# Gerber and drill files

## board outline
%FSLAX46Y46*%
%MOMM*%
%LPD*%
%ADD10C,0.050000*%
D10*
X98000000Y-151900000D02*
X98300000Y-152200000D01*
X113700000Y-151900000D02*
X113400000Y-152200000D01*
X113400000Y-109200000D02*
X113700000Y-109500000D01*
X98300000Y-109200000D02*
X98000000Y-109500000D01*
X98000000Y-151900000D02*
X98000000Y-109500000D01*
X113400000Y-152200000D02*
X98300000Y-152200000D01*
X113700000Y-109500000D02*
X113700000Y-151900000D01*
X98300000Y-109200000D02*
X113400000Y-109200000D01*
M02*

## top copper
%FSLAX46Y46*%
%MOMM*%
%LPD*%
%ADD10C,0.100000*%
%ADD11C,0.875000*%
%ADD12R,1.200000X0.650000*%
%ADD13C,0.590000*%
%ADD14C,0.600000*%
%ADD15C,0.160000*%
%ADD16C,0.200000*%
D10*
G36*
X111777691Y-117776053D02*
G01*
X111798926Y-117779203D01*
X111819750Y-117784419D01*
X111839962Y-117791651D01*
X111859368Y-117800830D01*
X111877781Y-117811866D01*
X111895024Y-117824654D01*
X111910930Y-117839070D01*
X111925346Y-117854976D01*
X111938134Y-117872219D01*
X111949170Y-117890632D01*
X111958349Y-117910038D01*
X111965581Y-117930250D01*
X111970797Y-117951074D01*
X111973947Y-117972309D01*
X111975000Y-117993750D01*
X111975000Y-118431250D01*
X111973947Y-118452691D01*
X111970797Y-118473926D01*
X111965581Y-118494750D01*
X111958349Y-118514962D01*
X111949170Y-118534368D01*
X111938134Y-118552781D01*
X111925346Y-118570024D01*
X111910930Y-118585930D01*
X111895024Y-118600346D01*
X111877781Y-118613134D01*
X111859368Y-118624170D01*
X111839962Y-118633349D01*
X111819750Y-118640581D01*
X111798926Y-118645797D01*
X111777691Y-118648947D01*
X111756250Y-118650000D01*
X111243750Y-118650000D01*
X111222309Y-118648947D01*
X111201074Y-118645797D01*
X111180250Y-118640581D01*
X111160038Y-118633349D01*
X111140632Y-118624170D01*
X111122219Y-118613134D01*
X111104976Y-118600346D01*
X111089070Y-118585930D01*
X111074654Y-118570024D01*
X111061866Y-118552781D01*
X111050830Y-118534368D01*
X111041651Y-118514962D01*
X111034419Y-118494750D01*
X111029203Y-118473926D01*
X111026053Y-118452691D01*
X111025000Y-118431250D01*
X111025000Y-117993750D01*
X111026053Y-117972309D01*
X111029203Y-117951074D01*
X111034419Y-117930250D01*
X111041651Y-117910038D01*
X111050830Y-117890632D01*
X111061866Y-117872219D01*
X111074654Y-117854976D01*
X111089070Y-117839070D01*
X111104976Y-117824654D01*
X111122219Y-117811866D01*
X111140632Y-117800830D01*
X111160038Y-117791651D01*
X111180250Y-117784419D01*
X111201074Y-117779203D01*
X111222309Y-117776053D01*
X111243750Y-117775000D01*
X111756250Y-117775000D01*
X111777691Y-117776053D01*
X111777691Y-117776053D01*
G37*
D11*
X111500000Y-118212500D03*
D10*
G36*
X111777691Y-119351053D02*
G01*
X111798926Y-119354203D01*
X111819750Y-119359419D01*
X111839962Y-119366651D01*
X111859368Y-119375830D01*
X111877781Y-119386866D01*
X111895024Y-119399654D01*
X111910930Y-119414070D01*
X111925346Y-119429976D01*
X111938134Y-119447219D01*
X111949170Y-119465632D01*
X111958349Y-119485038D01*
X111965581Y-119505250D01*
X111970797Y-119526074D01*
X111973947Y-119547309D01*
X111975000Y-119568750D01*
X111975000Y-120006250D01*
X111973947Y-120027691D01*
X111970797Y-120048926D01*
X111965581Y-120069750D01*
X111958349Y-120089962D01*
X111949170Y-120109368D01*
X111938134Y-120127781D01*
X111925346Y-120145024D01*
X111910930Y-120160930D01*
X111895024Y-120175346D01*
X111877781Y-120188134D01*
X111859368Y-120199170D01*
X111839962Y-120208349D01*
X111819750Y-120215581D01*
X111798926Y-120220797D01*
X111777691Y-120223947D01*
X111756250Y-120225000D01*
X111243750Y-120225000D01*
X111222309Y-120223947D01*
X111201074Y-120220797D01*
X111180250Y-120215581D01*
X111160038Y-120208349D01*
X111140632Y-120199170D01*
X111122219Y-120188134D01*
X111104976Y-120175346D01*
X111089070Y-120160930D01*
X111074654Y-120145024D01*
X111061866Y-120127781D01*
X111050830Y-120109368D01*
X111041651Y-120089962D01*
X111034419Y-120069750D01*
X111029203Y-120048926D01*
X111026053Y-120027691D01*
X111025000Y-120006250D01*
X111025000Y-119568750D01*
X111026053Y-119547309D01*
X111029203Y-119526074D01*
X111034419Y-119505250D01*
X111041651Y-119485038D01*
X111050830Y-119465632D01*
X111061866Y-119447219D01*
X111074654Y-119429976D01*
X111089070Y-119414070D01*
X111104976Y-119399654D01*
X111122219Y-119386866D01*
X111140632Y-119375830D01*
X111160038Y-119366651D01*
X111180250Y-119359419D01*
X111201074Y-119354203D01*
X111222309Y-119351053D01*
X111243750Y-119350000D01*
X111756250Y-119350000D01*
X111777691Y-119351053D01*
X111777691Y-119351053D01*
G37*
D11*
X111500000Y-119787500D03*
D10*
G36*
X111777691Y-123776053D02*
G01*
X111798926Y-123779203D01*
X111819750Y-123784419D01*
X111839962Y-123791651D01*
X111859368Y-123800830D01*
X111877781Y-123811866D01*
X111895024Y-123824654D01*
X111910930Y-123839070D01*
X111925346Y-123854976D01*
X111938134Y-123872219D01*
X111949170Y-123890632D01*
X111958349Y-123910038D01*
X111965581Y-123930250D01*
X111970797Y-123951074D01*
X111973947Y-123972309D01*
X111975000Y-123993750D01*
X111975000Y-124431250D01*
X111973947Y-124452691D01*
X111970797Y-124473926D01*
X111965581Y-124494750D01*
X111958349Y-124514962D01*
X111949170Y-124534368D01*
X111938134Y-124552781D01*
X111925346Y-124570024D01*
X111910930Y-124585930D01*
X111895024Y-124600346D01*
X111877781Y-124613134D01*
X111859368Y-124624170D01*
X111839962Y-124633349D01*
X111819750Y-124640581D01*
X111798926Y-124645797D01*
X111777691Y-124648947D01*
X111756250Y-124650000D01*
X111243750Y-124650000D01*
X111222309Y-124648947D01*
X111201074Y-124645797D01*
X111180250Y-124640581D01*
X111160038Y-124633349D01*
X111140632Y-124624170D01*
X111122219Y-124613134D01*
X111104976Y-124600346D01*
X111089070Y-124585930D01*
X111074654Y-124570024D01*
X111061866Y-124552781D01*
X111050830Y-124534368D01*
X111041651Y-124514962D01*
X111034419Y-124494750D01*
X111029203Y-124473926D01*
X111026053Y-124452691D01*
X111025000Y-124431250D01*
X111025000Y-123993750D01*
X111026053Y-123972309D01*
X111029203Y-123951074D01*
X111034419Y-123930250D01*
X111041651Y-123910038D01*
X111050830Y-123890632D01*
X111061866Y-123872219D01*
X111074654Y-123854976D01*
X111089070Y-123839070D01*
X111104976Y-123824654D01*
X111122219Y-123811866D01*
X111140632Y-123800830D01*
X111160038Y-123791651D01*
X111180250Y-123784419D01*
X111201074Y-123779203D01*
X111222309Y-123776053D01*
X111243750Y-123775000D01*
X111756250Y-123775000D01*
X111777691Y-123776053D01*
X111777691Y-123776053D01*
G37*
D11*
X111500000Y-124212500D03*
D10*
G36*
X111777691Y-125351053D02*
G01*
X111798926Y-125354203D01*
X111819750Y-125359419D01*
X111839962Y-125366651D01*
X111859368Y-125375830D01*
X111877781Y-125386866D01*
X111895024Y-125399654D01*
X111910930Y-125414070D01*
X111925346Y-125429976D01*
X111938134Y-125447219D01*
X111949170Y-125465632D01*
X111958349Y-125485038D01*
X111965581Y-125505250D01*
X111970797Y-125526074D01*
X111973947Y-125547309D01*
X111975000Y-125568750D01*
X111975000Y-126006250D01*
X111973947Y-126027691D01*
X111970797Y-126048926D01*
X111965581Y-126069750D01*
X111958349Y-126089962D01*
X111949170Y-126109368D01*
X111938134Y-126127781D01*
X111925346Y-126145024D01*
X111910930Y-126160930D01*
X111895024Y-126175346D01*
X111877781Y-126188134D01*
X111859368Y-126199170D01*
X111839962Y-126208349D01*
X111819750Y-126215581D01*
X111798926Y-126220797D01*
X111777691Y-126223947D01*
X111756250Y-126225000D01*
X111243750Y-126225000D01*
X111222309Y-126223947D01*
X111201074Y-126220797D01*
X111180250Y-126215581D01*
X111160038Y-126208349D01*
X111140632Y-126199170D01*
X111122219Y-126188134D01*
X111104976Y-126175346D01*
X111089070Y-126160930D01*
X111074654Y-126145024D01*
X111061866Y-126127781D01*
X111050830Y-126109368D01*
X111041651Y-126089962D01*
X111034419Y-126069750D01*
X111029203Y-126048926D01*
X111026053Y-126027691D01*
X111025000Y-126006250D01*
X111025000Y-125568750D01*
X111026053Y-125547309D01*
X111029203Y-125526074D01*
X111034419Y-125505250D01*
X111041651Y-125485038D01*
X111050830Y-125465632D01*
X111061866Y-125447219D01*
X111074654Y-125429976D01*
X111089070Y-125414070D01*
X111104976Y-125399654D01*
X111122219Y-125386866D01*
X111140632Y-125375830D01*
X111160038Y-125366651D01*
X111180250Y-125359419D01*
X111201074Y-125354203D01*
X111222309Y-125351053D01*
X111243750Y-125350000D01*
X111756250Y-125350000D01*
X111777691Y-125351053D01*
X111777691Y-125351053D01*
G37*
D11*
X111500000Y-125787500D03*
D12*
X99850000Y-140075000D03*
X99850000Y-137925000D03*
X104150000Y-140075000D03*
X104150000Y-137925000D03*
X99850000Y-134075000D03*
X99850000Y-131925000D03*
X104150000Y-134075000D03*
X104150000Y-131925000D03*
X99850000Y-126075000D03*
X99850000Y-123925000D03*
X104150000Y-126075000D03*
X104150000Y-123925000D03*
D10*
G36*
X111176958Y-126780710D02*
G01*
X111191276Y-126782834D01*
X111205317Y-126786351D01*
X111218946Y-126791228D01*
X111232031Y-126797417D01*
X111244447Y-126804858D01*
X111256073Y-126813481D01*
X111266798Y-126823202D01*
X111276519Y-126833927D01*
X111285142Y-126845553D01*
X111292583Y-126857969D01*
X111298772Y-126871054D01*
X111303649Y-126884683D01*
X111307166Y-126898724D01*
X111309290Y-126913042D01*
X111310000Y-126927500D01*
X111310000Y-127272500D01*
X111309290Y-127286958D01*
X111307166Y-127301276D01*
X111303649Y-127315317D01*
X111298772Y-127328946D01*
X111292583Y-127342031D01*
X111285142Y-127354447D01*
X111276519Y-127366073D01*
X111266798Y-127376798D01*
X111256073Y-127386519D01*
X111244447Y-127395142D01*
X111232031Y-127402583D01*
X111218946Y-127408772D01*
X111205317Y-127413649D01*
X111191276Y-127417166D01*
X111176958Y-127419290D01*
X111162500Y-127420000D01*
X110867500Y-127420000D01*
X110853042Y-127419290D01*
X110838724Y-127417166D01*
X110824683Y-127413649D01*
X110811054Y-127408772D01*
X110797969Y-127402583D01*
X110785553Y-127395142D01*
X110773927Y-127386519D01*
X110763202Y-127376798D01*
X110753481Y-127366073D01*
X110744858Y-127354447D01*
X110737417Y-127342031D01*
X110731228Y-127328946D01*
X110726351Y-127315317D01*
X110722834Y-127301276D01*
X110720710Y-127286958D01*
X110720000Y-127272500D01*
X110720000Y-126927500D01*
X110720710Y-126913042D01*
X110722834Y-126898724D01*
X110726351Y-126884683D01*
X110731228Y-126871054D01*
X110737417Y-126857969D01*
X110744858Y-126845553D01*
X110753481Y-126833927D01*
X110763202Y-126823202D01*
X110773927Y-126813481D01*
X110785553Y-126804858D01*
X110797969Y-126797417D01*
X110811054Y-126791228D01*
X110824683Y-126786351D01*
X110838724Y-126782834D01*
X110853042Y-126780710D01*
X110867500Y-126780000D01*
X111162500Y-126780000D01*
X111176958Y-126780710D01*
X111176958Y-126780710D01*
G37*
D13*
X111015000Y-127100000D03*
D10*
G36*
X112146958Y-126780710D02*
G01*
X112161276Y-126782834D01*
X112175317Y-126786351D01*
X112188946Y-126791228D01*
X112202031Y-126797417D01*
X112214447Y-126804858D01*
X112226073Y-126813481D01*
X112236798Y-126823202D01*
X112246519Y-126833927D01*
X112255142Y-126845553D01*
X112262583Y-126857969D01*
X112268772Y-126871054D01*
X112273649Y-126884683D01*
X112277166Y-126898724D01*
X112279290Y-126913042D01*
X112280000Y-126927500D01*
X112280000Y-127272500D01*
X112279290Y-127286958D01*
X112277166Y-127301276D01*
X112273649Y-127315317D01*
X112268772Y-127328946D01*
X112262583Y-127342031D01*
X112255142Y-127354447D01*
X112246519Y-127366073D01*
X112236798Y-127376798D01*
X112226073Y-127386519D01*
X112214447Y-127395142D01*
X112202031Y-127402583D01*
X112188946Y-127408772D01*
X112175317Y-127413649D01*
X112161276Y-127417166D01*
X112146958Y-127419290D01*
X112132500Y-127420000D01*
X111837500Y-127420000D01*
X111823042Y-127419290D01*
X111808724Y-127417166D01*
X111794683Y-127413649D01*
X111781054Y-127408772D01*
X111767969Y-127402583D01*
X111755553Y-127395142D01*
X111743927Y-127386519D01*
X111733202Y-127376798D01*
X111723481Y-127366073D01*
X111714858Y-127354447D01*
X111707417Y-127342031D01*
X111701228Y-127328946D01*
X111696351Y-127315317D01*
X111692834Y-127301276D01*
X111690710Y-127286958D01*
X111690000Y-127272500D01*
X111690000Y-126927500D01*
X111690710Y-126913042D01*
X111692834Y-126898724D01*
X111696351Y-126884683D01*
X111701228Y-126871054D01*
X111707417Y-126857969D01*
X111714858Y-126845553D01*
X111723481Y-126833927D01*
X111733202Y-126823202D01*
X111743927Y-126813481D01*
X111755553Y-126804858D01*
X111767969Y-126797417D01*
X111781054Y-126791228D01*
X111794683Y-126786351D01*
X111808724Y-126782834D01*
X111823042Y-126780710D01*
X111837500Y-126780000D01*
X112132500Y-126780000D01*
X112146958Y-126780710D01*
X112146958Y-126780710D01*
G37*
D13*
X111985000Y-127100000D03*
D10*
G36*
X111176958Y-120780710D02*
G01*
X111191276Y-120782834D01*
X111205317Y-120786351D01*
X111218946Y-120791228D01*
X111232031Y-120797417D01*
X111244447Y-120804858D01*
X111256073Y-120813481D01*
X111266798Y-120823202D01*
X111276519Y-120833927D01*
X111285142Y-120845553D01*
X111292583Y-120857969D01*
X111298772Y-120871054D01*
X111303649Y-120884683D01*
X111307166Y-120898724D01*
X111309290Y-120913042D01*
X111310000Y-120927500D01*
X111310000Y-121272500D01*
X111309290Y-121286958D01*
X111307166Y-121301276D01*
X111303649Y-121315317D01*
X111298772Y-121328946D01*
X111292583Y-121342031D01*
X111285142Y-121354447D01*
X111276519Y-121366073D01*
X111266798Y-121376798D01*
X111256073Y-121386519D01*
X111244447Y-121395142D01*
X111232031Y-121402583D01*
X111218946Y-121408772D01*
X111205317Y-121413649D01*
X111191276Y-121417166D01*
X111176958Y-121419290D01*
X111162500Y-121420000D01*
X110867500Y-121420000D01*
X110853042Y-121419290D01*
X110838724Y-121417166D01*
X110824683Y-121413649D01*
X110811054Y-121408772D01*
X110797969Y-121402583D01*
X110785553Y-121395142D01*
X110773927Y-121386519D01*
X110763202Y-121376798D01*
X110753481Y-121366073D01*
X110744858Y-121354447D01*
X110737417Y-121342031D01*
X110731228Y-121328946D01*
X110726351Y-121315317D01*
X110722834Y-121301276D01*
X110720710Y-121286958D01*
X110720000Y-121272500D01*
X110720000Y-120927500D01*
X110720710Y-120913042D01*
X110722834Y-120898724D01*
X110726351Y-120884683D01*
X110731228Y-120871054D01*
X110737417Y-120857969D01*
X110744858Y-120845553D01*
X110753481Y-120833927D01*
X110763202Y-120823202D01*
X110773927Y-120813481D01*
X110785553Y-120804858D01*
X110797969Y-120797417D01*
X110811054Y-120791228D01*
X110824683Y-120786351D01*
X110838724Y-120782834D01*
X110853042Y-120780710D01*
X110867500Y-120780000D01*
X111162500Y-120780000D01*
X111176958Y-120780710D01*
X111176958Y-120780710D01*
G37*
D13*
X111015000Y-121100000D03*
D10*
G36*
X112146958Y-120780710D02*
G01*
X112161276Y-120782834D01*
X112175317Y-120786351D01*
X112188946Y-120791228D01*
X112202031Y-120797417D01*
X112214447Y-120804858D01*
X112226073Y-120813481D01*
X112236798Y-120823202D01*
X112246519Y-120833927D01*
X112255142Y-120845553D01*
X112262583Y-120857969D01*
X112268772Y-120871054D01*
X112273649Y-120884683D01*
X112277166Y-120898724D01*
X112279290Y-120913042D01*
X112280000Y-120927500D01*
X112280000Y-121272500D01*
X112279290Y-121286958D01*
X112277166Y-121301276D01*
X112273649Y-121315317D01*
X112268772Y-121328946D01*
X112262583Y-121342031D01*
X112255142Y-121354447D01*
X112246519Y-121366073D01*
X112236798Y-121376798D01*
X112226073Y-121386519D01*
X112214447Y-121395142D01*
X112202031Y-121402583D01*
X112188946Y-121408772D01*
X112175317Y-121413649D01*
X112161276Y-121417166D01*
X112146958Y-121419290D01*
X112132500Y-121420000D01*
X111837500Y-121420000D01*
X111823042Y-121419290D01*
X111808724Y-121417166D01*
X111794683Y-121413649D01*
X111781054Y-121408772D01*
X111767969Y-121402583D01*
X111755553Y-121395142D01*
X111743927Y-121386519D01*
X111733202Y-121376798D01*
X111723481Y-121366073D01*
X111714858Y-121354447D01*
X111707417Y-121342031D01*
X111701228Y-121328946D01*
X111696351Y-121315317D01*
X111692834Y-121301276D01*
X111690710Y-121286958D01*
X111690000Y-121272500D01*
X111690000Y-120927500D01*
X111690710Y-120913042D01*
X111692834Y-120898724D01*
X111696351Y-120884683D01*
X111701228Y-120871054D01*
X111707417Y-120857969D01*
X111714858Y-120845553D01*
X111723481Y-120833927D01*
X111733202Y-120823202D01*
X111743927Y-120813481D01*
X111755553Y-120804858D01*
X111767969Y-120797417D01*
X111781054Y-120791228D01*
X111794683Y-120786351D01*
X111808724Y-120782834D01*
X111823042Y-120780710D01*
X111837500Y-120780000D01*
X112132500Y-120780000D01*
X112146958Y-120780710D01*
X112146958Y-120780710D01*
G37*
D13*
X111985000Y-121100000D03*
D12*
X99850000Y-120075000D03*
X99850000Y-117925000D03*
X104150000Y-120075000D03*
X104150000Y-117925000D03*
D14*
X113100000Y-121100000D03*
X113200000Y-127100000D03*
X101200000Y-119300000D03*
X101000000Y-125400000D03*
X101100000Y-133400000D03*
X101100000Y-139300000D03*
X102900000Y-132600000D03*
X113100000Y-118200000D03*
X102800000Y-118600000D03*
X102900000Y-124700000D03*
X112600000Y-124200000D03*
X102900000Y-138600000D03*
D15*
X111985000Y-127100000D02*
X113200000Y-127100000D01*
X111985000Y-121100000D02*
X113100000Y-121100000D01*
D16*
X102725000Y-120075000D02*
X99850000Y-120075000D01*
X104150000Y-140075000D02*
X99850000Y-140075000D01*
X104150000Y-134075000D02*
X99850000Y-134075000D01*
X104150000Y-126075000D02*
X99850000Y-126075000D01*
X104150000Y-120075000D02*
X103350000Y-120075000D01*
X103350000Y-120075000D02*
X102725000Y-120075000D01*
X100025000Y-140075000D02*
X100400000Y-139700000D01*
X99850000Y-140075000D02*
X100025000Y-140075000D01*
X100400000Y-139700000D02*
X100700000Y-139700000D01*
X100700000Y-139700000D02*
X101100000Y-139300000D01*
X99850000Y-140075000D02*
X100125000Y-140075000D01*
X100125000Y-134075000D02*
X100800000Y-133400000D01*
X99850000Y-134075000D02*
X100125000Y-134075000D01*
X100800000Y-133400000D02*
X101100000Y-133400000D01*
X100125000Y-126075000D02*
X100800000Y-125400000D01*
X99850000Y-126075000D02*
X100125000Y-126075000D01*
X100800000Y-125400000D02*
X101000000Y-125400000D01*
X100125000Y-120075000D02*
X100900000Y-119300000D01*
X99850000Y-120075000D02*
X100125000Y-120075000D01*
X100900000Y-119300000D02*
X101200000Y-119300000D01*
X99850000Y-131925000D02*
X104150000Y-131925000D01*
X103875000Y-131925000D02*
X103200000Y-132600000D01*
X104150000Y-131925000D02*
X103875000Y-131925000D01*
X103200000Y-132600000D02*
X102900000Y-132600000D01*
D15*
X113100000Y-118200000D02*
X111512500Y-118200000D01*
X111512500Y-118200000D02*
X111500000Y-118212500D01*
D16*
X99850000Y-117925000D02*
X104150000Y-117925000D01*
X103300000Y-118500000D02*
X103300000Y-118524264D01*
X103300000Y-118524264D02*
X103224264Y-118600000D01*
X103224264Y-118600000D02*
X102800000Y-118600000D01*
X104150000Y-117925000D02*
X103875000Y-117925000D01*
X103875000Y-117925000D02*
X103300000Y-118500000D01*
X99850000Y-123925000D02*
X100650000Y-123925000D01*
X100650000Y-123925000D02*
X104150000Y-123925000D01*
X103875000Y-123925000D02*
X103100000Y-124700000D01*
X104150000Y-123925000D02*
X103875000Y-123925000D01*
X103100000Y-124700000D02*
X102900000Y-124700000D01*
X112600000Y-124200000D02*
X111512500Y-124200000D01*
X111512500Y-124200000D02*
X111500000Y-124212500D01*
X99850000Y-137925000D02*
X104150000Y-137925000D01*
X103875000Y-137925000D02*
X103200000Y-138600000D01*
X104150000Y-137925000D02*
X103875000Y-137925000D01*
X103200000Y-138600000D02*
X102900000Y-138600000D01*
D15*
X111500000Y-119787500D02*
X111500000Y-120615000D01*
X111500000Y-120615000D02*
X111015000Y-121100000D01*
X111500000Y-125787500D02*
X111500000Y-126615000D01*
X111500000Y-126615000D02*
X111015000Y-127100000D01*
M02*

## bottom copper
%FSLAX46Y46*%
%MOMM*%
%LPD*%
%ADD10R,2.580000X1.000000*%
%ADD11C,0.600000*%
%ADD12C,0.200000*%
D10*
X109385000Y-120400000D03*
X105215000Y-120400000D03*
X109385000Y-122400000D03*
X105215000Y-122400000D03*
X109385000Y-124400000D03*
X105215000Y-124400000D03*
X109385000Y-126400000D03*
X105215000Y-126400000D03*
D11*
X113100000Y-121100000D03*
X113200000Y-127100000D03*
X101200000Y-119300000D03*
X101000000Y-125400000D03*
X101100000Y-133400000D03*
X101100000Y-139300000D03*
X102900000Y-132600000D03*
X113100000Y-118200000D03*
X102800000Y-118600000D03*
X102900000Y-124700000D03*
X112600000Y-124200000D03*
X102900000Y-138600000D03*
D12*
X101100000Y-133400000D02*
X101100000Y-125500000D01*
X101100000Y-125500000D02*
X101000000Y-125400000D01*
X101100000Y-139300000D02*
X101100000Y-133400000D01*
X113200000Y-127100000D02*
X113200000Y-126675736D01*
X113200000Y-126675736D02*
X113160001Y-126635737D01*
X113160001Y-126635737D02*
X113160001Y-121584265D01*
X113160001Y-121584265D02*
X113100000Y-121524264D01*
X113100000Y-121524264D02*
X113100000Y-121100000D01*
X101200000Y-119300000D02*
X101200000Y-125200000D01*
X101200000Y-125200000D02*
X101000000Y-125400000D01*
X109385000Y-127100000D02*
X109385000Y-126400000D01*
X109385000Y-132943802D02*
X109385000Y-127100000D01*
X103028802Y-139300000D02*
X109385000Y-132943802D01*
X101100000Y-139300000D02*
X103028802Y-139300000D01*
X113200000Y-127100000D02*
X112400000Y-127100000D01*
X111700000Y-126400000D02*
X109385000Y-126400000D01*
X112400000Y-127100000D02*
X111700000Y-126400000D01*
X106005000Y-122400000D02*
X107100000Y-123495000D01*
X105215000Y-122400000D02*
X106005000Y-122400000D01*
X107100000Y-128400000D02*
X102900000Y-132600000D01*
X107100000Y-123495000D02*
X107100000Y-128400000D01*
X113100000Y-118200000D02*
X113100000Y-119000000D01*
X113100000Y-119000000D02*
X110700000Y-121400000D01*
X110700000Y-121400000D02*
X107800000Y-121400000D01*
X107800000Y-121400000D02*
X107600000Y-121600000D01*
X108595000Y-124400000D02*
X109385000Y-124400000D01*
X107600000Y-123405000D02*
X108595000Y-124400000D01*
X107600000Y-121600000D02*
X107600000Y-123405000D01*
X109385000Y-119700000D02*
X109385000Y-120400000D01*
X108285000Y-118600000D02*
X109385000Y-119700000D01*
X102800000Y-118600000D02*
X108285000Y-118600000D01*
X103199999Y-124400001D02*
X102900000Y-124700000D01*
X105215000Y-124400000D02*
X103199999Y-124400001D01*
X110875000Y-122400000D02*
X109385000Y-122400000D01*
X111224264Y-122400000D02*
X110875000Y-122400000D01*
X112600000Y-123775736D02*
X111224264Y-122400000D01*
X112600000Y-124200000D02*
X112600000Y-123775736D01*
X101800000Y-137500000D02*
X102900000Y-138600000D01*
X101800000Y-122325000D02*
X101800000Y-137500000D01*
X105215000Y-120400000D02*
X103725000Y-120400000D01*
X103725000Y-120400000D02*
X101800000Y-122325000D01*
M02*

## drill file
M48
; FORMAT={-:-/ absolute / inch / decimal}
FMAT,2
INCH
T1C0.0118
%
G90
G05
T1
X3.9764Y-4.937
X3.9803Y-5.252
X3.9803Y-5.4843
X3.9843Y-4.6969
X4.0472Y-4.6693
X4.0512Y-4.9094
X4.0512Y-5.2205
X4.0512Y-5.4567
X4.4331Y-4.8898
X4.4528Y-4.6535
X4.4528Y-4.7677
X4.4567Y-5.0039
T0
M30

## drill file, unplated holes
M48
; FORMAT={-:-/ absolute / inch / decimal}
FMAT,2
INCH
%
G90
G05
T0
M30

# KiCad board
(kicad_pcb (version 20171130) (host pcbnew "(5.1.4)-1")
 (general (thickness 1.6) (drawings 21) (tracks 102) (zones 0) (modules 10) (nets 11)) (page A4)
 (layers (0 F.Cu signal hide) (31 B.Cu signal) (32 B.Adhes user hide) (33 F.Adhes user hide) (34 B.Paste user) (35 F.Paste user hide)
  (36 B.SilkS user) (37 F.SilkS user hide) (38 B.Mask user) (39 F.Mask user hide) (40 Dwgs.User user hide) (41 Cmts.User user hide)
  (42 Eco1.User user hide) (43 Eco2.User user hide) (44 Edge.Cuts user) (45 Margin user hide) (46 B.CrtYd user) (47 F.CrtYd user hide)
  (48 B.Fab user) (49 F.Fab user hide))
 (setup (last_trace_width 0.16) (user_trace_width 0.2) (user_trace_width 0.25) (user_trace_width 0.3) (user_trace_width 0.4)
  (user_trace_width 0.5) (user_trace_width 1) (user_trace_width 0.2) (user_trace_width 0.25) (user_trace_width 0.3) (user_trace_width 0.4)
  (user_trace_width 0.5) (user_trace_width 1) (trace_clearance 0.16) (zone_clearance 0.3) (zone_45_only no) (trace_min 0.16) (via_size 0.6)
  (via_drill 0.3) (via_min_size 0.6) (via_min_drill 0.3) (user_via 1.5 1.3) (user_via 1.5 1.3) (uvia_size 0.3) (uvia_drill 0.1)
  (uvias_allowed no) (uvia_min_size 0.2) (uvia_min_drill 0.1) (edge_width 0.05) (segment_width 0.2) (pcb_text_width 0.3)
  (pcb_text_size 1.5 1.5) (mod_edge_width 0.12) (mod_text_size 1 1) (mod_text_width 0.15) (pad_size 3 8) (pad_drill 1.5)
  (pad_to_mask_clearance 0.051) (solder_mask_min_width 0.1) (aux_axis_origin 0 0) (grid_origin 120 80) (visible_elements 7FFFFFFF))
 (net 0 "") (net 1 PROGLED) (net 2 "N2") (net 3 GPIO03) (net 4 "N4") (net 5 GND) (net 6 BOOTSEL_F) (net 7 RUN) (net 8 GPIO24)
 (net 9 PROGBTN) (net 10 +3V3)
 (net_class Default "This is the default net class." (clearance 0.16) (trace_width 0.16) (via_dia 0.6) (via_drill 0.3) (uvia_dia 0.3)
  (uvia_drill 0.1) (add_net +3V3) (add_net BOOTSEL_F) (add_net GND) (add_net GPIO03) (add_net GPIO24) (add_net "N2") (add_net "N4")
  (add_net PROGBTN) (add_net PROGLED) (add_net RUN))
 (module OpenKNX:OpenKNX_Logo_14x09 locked (layer F.Cu) (at 105.8 146.4)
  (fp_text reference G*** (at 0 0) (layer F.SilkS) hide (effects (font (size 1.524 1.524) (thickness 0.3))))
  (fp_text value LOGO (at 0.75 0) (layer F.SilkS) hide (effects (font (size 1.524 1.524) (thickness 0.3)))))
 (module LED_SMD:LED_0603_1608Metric (layer F.Cu) (at 111.5 119 90)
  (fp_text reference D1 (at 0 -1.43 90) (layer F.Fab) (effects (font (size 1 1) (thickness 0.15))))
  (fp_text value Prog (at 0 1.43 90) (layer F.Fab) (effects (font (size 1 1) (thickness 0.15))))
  (pad 2 smd roundrect (at 0.7875 0 90) (size 0.875 0.95) (layers F.Cu F.Paste F.Mask) (roundrect_rratio 0.25) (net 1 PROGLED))
  (pad 1 smd roundrect (at -0.7875 0 90) (size 0.875 0.95) (layers F.Cu F.Paste F.Mask) (roundrect_rratio 0.25) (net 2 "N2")))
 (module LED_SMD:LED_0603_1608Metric (layer F.Cu) (at 111.5 125 90)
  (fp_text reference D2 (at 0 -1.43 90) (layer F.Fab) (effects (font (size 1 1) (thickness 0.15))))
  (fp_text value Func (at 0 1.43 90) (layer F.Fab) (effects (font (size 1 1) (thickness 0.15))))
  (pad 2 smd roundrect (at 0.7875 0 90) (size 0.875 0.95) (layers F.Cu F.Paste F.Mask) (roundrect_rratio 0.25) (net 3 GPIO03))
  (pad 1 smd roundrect (at -0.7875 0 90) (size 0.875 0.95) (layers F.Cu F.Paste F.Mask) (roundrect_rratio 0.25) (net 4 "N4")))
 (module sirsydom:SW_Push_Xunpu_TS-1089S (layer F.Cu) (at 102 139)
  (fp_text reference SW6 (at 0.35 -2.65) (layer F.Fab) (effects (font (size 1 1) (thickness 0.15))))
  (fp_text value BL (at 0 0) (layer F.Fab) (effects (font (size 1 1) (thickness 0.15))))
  (pad 2 smd rect (at -2.15 1.075) (size 1.2 0.65) (layers F.Cu F.Paste F.Mask) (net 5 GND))
  (pad 1 smd rect (at -2.15 -1.075) (size 1.2 0.65) (layers F.Cu F.Paste F.Mask) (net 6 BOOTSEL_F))
  (pad 2 smd rect (at 2.15 1.075) (size 1.2 0.65) (layers F.Cu F.Paste F.Mask) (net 5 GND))
  (pad 1 smd rect (at 2.15 -1.075) (size 1.2 0.65) (layers F.Cu F.Paste F.Mask) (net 6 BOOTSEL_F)))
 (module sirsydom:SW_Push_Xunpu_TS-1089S (layer F.Cu) (at 102 133)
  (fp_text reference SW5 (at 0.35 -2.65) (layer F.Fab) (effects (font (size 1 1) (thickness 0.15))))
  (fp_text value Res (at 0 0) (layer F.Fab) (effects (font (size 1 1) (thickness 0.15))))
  (pad 2 smd rect (at -2.15 1.075) (size 1.2 0.65) (layers F.Cu F.Paste F.Mask) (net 5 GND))
  (pad 1 smd rect (at -2.15 -1.075) (size 1.2 0.65) (layers F.Cu F.Paste F.Mask) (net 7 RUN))
  (pad 2 smd rect (at 2.15 1.075) (size 1.2 0.65) (layers F.Cu F.Paste F.Mask) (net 5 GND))
  (pad 1 smd rect (at 2.15 -1.075) (size 1.2 0.65) (layers F.Cu F.Paste F.Mask) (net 7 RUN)))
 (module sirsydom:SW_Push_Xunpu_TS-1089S (layer F.Cu) (at 102 125)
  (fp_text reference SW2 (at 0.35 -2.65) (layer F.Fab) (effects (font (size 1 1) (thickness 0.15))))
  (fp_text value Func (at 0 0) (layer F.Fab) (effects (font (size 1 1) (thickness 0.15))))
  (pad 2 smd rect (at -2.15 1.075) (size 1.2 0.65) (layers F.Cu F.Paste F.Mask) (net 5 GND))
  (pad 1 smd rect (at -2.15 -1.075) (size 1.2 0.65) (layers F.Cu F.Paste F.Mask) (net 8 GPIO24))
  (pad 2 smd rect (at 2.15 1.075) (size 1.2 0.65) (layers F.Cu F.Paste F.Mask) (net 5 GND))
  (pad 1 smd rect (at 2.15 -1.075) (size 1.2 0.65) (layers F.Cu F.Paste F.Mask) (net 8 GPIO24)))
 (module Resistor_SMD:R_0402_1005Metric (layer F.Cu) (at 111.5 127.1 180)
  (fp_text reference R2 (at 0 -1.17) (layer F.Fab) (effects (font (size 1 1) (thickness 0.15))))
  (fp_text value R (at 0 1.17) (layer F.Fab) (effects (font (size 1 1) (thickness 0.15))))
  (pad 2 smd roundrect (at 0.485 0 180) (size 0.59 0.64) (layers F.Cu F.Paste F.Mask) (roundrect_rratio 0.25) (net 4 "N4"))
  (pad 1 smd roundrect (at -0.485 0 180) (size 0.59 0.64) (layers F.Cu F.Paste F.Mask) (roundrect_rratio 0.25) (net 5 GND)))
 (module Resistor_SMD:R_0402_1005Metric (layer F.Cu) (at 111.5 121.1 180)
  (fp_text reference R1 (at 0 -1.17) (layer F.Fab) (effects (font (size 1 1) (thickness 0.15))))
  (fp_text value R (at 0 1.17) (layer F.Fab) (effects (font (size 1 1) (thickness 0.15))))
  (pad 2 smd roundrect (at 0.485 0 180) (size 0.59 0.64) (layers F.Cu F.Paste F.Mask) (roundrect_rratio 0.25) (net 2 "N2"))
  (pad 1 smd roundrect (at -0.485 0 180) (size 0.59 0.64) (layers F.Cu F.Paste F.Mask) (roundrect_rratio 0.25) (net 5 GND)))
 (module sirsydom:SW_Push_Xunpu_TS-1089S (layer F.Cu) (at 102 119)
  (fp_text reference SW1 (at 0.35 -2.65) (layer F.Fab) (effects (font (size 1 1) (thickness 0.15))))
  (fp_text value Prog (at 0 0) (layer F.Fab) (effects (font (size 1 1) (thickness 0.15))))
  (pad 2 smd rect (at -2.15 1.075) (size 1.2 0.65) (layers F.Cu F.Paste F.Mask) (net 5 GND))
  (pad 1 smd rect (at -2.15 -1.075) (size 1.2 0.65) (layers F.Cu F.Paste F.Mask) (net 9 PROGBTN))
  (pad 2 smd rect (at 2.15 1.075) (size 1.2 0.65) (layers F.Cu F.Paste F.Mask) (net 5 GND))
  (pad 1 smd rect (at 2.15 -1.075) (size 1.2 0.65) (layers F.Cu F.Paste F.Mask) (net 9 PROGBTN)))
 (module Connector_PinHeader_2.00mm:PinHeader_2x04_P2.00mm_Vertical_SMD (layer B.Cu) (at 107.3 123.4)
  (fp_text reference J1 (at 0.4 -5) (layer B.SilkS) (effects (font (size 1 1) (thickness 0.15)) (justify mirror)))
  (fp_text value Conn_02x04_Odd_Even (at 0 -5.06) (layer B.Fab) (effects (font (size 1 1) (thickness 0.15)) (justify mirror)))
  (pad 8 smd rect (at 2.085 -3) (size 2.58 1) (layers B.Cu B.Paste B.Mask) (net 9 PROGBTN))
  (pad 7 smd rect (at -2.085 -3) (size 2.58 1) (layers B.Cu B.Paste B.Mask) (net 6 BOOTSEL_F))
  (pad 6 smd rect (at 2.085 -1) (size 2.58 1) (layers B.Cu B.Paste B.Mask) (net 3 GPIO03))
  (pad 5 smd rect (at -2.085 -1) (size 2.58 1) (layers B.Cu B.Paste B.Mask) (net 7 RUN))
  (pad 4 smd rect (at 2.085 1) (size 2.58 1) (layers B.Cu B.Paste B.Mask) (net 1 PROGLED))
  (pad 3 smd rect (at -2.085 1) (size 2.58 1) (layers B.Cu B.Paste B.Mask) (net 8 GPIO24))
  (pad 2 smd rect (at 2.085 3) (size 2.58 1) (layers B.Cu B.Paste B.Mask) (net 5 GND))
  (pad 1 smd rect (at -2.085 3) (size 2.58 1) (layers B.Cu B.Paste B.Mask) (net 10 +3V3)))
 (gr_line (start 98 151.9) (end 98.3 152.2) (layer Edge.Cuts) (width 0.05))
 (gr_line (start 113.7 151.9) (end 113.4 152.2) (layer Edge.Cuts) (width 0.05))
 (gr_line (start 113.4 109.2) (end 113.7 109.5) (layer Edge.Cuts) (width 0.05))
 (gr_line (start 98.3 109.2) (end 98 109.5) (layer Edge.Cuts) (width 0.05))
 (gr_line (start 98 151.9) (end 98 109.5) (layer Edge.Cuts) (width 0.05))
 (gr_line (start 113.4 152.2) (end 98.3 152.2) (layer Edge.Cuts) (width 0.05))
 (gr_line (start 113.7 109.5) (end 113.7 151.9) (layer Edge.Cuts) (width 0.05))
 (gr_line (start 98.3 109.2) (end 113.4 109.2) (layer Edge.Cuts) (width 0.05))
 (segment (start 101.1 133.4) (end 101.1 125.5) (width 0.2) (layer B.Cu) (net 5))
 (segment (start 101.1 125.5) (end 101 125.4) (width 0.2) (layer B.Cu) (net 5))
 (segment (start 101.1 139.3) (end 101.1 133.4) (width 0.2) (layer B.Cu) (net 5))
 (segment (start 113.2 127.1) (end 113.2 126.675736) (width 0.2) (layer B.Cu) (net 5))
 (segment (start 113.2 126.675736) (end 113.160001 126.635737) (width 0.2) (layer B.Cu) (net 5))
 (segment (start 113.160001 126.635737) (end 113.160001 121.584265) (width 0.2) (layer B.Cu) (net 5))
 (segment (start 113.160001 121.584265) (end 113.1 121.524264) (width 0.2) (layer B.Cu) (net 5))
 (segment (start 113.1 121.524264) (end 113.1 121.1) (width 0.2) (layer B.Cu) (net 5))
 (segment (start 111.985 127.1) (end 113.2 127.1) (width 0.16) (layer F.Cu) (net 5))
 (segment (start 111.985 121.1) (end 113.1 121.1) (width 0.16) (layer F.Cu) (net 5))
 (via (at 113.1 121.1) (size 0.6) (drill 0.3) (layers F.Cu B.Cu) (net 5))
 (via (at 113.2 127.1) (size 0.6) (drill 0.3) (layers F.Cu B.Cu) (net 5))
 (segment (start 102.725 120.075) (end 99.85 120.075) (width 0.2) (layer F.Cu) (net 5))
 (segment (start 104.15 140.075) (end 99.85 140.075) (width 0.2) (layer F.Cu) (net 5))
 (segment (start 104.15 134.075) (end 99.85 134.075) (width 0.2) (layer F.Cu) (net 5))
 (segment (start 104.15 126.075) (end 99.85 126.075) (width 0.2) (layer F.Cu) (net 5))
 (segment (start 104.15 120.075) (end 103.35 120.075) (width 0.2) (layer F.Cu) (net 5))
 (segment (start 103.35 120.075) (end 102.725 120.075) (width 0.2) (layer F.Cu) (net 5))
 (segment (start 101.2 119.3) (end 101.2 125.2) (width 0.2) (layer B.Cu) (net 5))
 (segment (start 101.2 125.2) (end 101 125.4) (width 0.2) (layer B.Cu) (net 5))
 (segment (start 100.025 140.075) (end 100.4 139.7) (width 0.2) (layer F.Cu) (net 5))
 (segment (start 99.85 140.075) (end 100.025 140.075) (width 0.2) (layer F.Cu) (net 5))
 (segment (start 100.4 139.7) (end 100.7 139.7) (width 0.2) (layer F.Cu) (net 5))
 (segment (start 100.7 139.7) (end 101.1 139.3) (width 0.2) (layer F.Cu) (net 5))
 (segment (start 99.85 140.075) (end 100.125 140.075) (width 0.2) (layer F.Cu) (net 5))
 (segment (start 100.125 134.075) (end 100.8 133.4) (width 0.2) (layer F.Cu) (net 5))
 (segment (start 99.85 134.075) (end 100.125 134.075) (width 0.2) (layer F.Cu) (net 5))
 (segment (start 100.8 133.4) (end 101.1 133.4) (width 0.2) (layer F.Cu) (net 5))
 (segment (start 100.125 126.075) (end 100.8 125.4) (width 0.2) (layer F.Cu) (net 5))
 (segment (start 99.85 126.075) (end 100.125 126.075) (width 0.2) (layer F.Cu) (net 5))
 (segment (start 100.8 125.4) (end 101 125.4) (width 0.2) (layer F.Cu) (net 5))
 (segment (start 100.125 120.075) (end 100.9 119.3) (width 0.2) (layer F.Cu) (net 5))
 (segment (start 99.85 120.075) (end 100.125 120.075) (width 0.2) (layer F.Cu) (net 5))
 (segment (start 100.9 119.3) (end 101.2 119.3) (width 0.2) (layer F.Cu) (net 5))
 (via (at 101.2 119.3) (size 0.6) (drill 0.3) (layers F.Cu B.Cu) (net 5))
 (via (at 101 125.4) (size 0.6) (drill 0.3) (layers F.Cu B.Cu) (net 5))
 (via (at 101.1 133.4) (size 0.6) (drill 0.3) (layers F.Cu B.Cu) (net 5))
 (via (at 101.1 139.3) (size 0.6) (drill 0.3) (layers F.Cu B.Cu) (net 5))
 (segment (start 109.385 127.1) (end 109.385 126.4) (width 0.2) (layer B.Cu) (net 5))
 (segment (start 109.385 132.943802) (end 109.385 127.1) (width 0.2) (layer B.Cu) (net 5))
 (segment (start 103.028802 139.3) (end 109.385 132.943802) (width 0.2) (layer B.Cu) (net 5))
 (segment (start 101.1 139.3) (end 103.028802 139.3) (width 0.2) (layer B.Cu) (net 5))
 (segment (start 113.2 127.1) (end 112.4 127.1) (width 0.2) (layer B.Cu) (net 5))
 (segment (start 111.7 126.4) (end 109.385 126.4) (width 0.2) (layer B.Cu) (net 5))
 (segment (start 112.4 127.1) (end 111.7 126.4) (width 0.2) (layer B.Cu) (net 5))
 (segment (start 99.85 131.925) (end 104.15 131.925) (width 0.2) (layer F.Cu) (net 7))
 (segment (start 103.875 131.925) (end 103.2 132.6) (width 0.2) (layer F.Cu) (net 7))
 (segment (start 104.15 131.925) (end 103.875 131.925) (width 0.2) (layer F.Cu) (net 7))
 (segment (start 103.2 132.6) (end 102.9 132.6) (width 0.2) (layer F.Cu) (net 7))
 (via (at 102.9 132.6) (size 0.6) (drill 0.3) (layers F.Cu B.Cu) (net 7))
 (segment (start 106.005 122.4) (end 107.1 123.495) (width 0.2) (layer B.Cu) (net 7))
 (segment (start 105.215 122.4) (end 106.005 122.4) (width 0.2) (layer B.Cu) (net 7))
 (segment (start 107.1 128.4) (end 102.9 132.6) (width 0.2) (layer B.Cu) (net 7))
 (segment (start 107.1 123.495) (end 107.1 128.4) (width 0.2) (layer B.Cu) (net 7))
 (segment (start 113.1 118.2) (end 111.5125 118.2) (width 0.16) (layer F.Cu) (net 1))
 (segment (start 111.5125 118.2) (end 111.5 118.2125) (width 0.16) (layer F.Cu) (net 1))
 (via (at 113.1 118.2) (size 0.6) (drill 0.3) (layers F.Cu B.Cu) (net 1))
 (segment (start 113.1 118.2) (end 113.1 119) (width 0.2) (layer B.Cu) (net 1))
 (segment (start 113.1 119) (end 110.7 121.4) (width 0.2) (layer B.Cu) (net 1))
 (segment (start 110.7 121.4) (end 107.8 121.4) (width 0.2) (layer B.Cu) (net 1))
 (segment (start 107.8 121.4) (end 107.6 121.6) (width 0.2) (layer B.Cu) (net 1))
 (segment (start 108.595 124.4) (end 109.385 124.4) (width 0.2) (layer B.Cu) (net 1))
 (segment (start 107.6 123.405) (end 108.595 124.4) (width 0.2) (layer B.Cu) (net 1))
 (segment (start 107.6 121.6) (end 107.6 123.405) (width 0.2) (layer B.Cu) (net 1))
 (segment (start 99.85 117.925) (end 104.15 117.925) (width 0.2) (layer F.Cu) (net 9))
 (segment (start 103.3 118.5) (end 103.3 118.524264) (width 0.2) (layer F.Cu) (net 9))
 (segment (start 103.3 118.524264) (end 103.224264 118.6) (width 0.2) (layer F.Cu) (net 9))
 (segment (start 103.224264 118.6) (end 102.8 118.6) (width 0.2) (layer F.Cu) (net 9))
 (segment (start 104.15 117.925) (end 103.875 117.925) (width 0.2) (layer F.Cu) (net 9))
 (segment (start 103.875 117.925) (end 103.3 118.5) (width 0.2) (layer F.Cu) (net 9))
 (via (at 102.8 118.6) (size 0.6) (drill 0.3) (layers F.Cu B.Cu) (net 9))
 (segment (start 109.385 119.7) (end 109.385 120.4) (width 0.2) (layer B.Cu) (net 9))
 (segment (start 108.285 118.6) (end 109.385 119.7) (width 0.2) (layer B.Cu) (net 9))
 (segment (start 102.8 118.6) (end 108.285 118.6) (width 0.2) (layer B.Cu) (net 9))
 (segment (start 99.85 123.925) (end 100.65 123.925) (width 0.2) (layer F.Cu) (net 8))
 (segment (start 100.65 123.925) (end 104.15 123.925) (width 0.2) (layer F.Cu) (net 8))
 (segment (start 103.875 123.925) (end 103.1 124.7) (width 0.2) (layer F.Cu) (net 8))
 (segment (start 104.15 123.925) (end 103.875 123.925) (width 0.2) (layer F.Cu) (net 8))
 (segment (start 103.1 124.7) (end 102.9 124.7) (width 0.2) (layer F.Cu) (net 8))
 (via (at 102.9 124.7) (size 0.6) (drill 0.3) (layers F.Cu B.Cu) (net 8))
 (segment (start 103.199999 124.400001) (end 102.9 124.7) (width 0.2) (layer B.Cu) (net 8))
 (segment (start 105.215 124.4) (end 103.199999 124.400001) (width 0.2) (layer B.Cu) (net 8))
 (segment (start 112.6 124.2) (end 111.5125 124.2) (width 0.2) (layer F.Cu) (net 3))
 (segment (start 111.5125 124.2) (end 111.5 124.2125) (width 0.2) (layer F.Cu) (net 3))
 (via (at 112.6 124.2) (size 0.6) (drill 0.3) (layers F.Cu B.Cu) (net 3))
 (segment (start 110.875 122.4) (end 109.385 122.4) (width 0.2) (layer B.Cu) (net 3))
 (segment (start 111.224264 122.4) (end 110.875 122.4) (width 0.2) (layer B.Cu) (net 3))
 (segment (start 112.6 123.775736) (end 111.224264 122.4) (width 0.2) (layer B.Cu) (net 3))
 (segment (start 112.6 124.2) (end 112.6 123.775736) (width 0.2) (layer B.Cu) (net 3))
 (segment (start 99.85 137.925) (end 104.15 137.925) (width 0.2) (layer F.Cu) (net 6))
 (segment (start 103.875 137.925) (end 103.2 138.6) (width 0.2) (layer F.Cu) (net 6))
 (segment (start 104.15 137.925) (end 103.875 137.925) (width 0.2) (layer F.Cu) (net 6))
 (segment (start 103.2 138.6) (end 102.9 138.6) (width 0.2) (layer F.Cu) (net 6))
 (via (at 102.9 138.6) (size 0.6) (drill 0.3) (layers F.Cu B.Cu) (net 6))
 (segment (start 101.8 137.5) (end 102.9 138.6) (width 0.2) (layer B.Cu) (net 6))
 (segment (start 101.8 122.325) (end 101.8 137.5) (width 0.2) (layer B.Cu) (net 6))
 (segment (start 105.215 120.4) (end 103.725 120.4) (width 0.2) (layer B.Cu) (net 6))
 (segment (start 103.725 120.4) (end 101.8 122.325) (width 0.2) (layer B.Cu) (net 6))
 (segment (start 111.5 119.7875) (end 111.5 120.615) (width 0.16) (layer F.Cu) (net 2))
 (segment (start 111.5 120.615) (end 111.015 121.1) (width 0.16) (layer F.Cu) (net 2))
 (segment (start 111.5 125.7875) (end 111.5 126.615) (width 0.16) (layer F.Cu) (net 4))
 (segment (start 111.5 126.615) (end 111.015 127.1) (width 0.16) (layer F.Cu) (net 4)))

